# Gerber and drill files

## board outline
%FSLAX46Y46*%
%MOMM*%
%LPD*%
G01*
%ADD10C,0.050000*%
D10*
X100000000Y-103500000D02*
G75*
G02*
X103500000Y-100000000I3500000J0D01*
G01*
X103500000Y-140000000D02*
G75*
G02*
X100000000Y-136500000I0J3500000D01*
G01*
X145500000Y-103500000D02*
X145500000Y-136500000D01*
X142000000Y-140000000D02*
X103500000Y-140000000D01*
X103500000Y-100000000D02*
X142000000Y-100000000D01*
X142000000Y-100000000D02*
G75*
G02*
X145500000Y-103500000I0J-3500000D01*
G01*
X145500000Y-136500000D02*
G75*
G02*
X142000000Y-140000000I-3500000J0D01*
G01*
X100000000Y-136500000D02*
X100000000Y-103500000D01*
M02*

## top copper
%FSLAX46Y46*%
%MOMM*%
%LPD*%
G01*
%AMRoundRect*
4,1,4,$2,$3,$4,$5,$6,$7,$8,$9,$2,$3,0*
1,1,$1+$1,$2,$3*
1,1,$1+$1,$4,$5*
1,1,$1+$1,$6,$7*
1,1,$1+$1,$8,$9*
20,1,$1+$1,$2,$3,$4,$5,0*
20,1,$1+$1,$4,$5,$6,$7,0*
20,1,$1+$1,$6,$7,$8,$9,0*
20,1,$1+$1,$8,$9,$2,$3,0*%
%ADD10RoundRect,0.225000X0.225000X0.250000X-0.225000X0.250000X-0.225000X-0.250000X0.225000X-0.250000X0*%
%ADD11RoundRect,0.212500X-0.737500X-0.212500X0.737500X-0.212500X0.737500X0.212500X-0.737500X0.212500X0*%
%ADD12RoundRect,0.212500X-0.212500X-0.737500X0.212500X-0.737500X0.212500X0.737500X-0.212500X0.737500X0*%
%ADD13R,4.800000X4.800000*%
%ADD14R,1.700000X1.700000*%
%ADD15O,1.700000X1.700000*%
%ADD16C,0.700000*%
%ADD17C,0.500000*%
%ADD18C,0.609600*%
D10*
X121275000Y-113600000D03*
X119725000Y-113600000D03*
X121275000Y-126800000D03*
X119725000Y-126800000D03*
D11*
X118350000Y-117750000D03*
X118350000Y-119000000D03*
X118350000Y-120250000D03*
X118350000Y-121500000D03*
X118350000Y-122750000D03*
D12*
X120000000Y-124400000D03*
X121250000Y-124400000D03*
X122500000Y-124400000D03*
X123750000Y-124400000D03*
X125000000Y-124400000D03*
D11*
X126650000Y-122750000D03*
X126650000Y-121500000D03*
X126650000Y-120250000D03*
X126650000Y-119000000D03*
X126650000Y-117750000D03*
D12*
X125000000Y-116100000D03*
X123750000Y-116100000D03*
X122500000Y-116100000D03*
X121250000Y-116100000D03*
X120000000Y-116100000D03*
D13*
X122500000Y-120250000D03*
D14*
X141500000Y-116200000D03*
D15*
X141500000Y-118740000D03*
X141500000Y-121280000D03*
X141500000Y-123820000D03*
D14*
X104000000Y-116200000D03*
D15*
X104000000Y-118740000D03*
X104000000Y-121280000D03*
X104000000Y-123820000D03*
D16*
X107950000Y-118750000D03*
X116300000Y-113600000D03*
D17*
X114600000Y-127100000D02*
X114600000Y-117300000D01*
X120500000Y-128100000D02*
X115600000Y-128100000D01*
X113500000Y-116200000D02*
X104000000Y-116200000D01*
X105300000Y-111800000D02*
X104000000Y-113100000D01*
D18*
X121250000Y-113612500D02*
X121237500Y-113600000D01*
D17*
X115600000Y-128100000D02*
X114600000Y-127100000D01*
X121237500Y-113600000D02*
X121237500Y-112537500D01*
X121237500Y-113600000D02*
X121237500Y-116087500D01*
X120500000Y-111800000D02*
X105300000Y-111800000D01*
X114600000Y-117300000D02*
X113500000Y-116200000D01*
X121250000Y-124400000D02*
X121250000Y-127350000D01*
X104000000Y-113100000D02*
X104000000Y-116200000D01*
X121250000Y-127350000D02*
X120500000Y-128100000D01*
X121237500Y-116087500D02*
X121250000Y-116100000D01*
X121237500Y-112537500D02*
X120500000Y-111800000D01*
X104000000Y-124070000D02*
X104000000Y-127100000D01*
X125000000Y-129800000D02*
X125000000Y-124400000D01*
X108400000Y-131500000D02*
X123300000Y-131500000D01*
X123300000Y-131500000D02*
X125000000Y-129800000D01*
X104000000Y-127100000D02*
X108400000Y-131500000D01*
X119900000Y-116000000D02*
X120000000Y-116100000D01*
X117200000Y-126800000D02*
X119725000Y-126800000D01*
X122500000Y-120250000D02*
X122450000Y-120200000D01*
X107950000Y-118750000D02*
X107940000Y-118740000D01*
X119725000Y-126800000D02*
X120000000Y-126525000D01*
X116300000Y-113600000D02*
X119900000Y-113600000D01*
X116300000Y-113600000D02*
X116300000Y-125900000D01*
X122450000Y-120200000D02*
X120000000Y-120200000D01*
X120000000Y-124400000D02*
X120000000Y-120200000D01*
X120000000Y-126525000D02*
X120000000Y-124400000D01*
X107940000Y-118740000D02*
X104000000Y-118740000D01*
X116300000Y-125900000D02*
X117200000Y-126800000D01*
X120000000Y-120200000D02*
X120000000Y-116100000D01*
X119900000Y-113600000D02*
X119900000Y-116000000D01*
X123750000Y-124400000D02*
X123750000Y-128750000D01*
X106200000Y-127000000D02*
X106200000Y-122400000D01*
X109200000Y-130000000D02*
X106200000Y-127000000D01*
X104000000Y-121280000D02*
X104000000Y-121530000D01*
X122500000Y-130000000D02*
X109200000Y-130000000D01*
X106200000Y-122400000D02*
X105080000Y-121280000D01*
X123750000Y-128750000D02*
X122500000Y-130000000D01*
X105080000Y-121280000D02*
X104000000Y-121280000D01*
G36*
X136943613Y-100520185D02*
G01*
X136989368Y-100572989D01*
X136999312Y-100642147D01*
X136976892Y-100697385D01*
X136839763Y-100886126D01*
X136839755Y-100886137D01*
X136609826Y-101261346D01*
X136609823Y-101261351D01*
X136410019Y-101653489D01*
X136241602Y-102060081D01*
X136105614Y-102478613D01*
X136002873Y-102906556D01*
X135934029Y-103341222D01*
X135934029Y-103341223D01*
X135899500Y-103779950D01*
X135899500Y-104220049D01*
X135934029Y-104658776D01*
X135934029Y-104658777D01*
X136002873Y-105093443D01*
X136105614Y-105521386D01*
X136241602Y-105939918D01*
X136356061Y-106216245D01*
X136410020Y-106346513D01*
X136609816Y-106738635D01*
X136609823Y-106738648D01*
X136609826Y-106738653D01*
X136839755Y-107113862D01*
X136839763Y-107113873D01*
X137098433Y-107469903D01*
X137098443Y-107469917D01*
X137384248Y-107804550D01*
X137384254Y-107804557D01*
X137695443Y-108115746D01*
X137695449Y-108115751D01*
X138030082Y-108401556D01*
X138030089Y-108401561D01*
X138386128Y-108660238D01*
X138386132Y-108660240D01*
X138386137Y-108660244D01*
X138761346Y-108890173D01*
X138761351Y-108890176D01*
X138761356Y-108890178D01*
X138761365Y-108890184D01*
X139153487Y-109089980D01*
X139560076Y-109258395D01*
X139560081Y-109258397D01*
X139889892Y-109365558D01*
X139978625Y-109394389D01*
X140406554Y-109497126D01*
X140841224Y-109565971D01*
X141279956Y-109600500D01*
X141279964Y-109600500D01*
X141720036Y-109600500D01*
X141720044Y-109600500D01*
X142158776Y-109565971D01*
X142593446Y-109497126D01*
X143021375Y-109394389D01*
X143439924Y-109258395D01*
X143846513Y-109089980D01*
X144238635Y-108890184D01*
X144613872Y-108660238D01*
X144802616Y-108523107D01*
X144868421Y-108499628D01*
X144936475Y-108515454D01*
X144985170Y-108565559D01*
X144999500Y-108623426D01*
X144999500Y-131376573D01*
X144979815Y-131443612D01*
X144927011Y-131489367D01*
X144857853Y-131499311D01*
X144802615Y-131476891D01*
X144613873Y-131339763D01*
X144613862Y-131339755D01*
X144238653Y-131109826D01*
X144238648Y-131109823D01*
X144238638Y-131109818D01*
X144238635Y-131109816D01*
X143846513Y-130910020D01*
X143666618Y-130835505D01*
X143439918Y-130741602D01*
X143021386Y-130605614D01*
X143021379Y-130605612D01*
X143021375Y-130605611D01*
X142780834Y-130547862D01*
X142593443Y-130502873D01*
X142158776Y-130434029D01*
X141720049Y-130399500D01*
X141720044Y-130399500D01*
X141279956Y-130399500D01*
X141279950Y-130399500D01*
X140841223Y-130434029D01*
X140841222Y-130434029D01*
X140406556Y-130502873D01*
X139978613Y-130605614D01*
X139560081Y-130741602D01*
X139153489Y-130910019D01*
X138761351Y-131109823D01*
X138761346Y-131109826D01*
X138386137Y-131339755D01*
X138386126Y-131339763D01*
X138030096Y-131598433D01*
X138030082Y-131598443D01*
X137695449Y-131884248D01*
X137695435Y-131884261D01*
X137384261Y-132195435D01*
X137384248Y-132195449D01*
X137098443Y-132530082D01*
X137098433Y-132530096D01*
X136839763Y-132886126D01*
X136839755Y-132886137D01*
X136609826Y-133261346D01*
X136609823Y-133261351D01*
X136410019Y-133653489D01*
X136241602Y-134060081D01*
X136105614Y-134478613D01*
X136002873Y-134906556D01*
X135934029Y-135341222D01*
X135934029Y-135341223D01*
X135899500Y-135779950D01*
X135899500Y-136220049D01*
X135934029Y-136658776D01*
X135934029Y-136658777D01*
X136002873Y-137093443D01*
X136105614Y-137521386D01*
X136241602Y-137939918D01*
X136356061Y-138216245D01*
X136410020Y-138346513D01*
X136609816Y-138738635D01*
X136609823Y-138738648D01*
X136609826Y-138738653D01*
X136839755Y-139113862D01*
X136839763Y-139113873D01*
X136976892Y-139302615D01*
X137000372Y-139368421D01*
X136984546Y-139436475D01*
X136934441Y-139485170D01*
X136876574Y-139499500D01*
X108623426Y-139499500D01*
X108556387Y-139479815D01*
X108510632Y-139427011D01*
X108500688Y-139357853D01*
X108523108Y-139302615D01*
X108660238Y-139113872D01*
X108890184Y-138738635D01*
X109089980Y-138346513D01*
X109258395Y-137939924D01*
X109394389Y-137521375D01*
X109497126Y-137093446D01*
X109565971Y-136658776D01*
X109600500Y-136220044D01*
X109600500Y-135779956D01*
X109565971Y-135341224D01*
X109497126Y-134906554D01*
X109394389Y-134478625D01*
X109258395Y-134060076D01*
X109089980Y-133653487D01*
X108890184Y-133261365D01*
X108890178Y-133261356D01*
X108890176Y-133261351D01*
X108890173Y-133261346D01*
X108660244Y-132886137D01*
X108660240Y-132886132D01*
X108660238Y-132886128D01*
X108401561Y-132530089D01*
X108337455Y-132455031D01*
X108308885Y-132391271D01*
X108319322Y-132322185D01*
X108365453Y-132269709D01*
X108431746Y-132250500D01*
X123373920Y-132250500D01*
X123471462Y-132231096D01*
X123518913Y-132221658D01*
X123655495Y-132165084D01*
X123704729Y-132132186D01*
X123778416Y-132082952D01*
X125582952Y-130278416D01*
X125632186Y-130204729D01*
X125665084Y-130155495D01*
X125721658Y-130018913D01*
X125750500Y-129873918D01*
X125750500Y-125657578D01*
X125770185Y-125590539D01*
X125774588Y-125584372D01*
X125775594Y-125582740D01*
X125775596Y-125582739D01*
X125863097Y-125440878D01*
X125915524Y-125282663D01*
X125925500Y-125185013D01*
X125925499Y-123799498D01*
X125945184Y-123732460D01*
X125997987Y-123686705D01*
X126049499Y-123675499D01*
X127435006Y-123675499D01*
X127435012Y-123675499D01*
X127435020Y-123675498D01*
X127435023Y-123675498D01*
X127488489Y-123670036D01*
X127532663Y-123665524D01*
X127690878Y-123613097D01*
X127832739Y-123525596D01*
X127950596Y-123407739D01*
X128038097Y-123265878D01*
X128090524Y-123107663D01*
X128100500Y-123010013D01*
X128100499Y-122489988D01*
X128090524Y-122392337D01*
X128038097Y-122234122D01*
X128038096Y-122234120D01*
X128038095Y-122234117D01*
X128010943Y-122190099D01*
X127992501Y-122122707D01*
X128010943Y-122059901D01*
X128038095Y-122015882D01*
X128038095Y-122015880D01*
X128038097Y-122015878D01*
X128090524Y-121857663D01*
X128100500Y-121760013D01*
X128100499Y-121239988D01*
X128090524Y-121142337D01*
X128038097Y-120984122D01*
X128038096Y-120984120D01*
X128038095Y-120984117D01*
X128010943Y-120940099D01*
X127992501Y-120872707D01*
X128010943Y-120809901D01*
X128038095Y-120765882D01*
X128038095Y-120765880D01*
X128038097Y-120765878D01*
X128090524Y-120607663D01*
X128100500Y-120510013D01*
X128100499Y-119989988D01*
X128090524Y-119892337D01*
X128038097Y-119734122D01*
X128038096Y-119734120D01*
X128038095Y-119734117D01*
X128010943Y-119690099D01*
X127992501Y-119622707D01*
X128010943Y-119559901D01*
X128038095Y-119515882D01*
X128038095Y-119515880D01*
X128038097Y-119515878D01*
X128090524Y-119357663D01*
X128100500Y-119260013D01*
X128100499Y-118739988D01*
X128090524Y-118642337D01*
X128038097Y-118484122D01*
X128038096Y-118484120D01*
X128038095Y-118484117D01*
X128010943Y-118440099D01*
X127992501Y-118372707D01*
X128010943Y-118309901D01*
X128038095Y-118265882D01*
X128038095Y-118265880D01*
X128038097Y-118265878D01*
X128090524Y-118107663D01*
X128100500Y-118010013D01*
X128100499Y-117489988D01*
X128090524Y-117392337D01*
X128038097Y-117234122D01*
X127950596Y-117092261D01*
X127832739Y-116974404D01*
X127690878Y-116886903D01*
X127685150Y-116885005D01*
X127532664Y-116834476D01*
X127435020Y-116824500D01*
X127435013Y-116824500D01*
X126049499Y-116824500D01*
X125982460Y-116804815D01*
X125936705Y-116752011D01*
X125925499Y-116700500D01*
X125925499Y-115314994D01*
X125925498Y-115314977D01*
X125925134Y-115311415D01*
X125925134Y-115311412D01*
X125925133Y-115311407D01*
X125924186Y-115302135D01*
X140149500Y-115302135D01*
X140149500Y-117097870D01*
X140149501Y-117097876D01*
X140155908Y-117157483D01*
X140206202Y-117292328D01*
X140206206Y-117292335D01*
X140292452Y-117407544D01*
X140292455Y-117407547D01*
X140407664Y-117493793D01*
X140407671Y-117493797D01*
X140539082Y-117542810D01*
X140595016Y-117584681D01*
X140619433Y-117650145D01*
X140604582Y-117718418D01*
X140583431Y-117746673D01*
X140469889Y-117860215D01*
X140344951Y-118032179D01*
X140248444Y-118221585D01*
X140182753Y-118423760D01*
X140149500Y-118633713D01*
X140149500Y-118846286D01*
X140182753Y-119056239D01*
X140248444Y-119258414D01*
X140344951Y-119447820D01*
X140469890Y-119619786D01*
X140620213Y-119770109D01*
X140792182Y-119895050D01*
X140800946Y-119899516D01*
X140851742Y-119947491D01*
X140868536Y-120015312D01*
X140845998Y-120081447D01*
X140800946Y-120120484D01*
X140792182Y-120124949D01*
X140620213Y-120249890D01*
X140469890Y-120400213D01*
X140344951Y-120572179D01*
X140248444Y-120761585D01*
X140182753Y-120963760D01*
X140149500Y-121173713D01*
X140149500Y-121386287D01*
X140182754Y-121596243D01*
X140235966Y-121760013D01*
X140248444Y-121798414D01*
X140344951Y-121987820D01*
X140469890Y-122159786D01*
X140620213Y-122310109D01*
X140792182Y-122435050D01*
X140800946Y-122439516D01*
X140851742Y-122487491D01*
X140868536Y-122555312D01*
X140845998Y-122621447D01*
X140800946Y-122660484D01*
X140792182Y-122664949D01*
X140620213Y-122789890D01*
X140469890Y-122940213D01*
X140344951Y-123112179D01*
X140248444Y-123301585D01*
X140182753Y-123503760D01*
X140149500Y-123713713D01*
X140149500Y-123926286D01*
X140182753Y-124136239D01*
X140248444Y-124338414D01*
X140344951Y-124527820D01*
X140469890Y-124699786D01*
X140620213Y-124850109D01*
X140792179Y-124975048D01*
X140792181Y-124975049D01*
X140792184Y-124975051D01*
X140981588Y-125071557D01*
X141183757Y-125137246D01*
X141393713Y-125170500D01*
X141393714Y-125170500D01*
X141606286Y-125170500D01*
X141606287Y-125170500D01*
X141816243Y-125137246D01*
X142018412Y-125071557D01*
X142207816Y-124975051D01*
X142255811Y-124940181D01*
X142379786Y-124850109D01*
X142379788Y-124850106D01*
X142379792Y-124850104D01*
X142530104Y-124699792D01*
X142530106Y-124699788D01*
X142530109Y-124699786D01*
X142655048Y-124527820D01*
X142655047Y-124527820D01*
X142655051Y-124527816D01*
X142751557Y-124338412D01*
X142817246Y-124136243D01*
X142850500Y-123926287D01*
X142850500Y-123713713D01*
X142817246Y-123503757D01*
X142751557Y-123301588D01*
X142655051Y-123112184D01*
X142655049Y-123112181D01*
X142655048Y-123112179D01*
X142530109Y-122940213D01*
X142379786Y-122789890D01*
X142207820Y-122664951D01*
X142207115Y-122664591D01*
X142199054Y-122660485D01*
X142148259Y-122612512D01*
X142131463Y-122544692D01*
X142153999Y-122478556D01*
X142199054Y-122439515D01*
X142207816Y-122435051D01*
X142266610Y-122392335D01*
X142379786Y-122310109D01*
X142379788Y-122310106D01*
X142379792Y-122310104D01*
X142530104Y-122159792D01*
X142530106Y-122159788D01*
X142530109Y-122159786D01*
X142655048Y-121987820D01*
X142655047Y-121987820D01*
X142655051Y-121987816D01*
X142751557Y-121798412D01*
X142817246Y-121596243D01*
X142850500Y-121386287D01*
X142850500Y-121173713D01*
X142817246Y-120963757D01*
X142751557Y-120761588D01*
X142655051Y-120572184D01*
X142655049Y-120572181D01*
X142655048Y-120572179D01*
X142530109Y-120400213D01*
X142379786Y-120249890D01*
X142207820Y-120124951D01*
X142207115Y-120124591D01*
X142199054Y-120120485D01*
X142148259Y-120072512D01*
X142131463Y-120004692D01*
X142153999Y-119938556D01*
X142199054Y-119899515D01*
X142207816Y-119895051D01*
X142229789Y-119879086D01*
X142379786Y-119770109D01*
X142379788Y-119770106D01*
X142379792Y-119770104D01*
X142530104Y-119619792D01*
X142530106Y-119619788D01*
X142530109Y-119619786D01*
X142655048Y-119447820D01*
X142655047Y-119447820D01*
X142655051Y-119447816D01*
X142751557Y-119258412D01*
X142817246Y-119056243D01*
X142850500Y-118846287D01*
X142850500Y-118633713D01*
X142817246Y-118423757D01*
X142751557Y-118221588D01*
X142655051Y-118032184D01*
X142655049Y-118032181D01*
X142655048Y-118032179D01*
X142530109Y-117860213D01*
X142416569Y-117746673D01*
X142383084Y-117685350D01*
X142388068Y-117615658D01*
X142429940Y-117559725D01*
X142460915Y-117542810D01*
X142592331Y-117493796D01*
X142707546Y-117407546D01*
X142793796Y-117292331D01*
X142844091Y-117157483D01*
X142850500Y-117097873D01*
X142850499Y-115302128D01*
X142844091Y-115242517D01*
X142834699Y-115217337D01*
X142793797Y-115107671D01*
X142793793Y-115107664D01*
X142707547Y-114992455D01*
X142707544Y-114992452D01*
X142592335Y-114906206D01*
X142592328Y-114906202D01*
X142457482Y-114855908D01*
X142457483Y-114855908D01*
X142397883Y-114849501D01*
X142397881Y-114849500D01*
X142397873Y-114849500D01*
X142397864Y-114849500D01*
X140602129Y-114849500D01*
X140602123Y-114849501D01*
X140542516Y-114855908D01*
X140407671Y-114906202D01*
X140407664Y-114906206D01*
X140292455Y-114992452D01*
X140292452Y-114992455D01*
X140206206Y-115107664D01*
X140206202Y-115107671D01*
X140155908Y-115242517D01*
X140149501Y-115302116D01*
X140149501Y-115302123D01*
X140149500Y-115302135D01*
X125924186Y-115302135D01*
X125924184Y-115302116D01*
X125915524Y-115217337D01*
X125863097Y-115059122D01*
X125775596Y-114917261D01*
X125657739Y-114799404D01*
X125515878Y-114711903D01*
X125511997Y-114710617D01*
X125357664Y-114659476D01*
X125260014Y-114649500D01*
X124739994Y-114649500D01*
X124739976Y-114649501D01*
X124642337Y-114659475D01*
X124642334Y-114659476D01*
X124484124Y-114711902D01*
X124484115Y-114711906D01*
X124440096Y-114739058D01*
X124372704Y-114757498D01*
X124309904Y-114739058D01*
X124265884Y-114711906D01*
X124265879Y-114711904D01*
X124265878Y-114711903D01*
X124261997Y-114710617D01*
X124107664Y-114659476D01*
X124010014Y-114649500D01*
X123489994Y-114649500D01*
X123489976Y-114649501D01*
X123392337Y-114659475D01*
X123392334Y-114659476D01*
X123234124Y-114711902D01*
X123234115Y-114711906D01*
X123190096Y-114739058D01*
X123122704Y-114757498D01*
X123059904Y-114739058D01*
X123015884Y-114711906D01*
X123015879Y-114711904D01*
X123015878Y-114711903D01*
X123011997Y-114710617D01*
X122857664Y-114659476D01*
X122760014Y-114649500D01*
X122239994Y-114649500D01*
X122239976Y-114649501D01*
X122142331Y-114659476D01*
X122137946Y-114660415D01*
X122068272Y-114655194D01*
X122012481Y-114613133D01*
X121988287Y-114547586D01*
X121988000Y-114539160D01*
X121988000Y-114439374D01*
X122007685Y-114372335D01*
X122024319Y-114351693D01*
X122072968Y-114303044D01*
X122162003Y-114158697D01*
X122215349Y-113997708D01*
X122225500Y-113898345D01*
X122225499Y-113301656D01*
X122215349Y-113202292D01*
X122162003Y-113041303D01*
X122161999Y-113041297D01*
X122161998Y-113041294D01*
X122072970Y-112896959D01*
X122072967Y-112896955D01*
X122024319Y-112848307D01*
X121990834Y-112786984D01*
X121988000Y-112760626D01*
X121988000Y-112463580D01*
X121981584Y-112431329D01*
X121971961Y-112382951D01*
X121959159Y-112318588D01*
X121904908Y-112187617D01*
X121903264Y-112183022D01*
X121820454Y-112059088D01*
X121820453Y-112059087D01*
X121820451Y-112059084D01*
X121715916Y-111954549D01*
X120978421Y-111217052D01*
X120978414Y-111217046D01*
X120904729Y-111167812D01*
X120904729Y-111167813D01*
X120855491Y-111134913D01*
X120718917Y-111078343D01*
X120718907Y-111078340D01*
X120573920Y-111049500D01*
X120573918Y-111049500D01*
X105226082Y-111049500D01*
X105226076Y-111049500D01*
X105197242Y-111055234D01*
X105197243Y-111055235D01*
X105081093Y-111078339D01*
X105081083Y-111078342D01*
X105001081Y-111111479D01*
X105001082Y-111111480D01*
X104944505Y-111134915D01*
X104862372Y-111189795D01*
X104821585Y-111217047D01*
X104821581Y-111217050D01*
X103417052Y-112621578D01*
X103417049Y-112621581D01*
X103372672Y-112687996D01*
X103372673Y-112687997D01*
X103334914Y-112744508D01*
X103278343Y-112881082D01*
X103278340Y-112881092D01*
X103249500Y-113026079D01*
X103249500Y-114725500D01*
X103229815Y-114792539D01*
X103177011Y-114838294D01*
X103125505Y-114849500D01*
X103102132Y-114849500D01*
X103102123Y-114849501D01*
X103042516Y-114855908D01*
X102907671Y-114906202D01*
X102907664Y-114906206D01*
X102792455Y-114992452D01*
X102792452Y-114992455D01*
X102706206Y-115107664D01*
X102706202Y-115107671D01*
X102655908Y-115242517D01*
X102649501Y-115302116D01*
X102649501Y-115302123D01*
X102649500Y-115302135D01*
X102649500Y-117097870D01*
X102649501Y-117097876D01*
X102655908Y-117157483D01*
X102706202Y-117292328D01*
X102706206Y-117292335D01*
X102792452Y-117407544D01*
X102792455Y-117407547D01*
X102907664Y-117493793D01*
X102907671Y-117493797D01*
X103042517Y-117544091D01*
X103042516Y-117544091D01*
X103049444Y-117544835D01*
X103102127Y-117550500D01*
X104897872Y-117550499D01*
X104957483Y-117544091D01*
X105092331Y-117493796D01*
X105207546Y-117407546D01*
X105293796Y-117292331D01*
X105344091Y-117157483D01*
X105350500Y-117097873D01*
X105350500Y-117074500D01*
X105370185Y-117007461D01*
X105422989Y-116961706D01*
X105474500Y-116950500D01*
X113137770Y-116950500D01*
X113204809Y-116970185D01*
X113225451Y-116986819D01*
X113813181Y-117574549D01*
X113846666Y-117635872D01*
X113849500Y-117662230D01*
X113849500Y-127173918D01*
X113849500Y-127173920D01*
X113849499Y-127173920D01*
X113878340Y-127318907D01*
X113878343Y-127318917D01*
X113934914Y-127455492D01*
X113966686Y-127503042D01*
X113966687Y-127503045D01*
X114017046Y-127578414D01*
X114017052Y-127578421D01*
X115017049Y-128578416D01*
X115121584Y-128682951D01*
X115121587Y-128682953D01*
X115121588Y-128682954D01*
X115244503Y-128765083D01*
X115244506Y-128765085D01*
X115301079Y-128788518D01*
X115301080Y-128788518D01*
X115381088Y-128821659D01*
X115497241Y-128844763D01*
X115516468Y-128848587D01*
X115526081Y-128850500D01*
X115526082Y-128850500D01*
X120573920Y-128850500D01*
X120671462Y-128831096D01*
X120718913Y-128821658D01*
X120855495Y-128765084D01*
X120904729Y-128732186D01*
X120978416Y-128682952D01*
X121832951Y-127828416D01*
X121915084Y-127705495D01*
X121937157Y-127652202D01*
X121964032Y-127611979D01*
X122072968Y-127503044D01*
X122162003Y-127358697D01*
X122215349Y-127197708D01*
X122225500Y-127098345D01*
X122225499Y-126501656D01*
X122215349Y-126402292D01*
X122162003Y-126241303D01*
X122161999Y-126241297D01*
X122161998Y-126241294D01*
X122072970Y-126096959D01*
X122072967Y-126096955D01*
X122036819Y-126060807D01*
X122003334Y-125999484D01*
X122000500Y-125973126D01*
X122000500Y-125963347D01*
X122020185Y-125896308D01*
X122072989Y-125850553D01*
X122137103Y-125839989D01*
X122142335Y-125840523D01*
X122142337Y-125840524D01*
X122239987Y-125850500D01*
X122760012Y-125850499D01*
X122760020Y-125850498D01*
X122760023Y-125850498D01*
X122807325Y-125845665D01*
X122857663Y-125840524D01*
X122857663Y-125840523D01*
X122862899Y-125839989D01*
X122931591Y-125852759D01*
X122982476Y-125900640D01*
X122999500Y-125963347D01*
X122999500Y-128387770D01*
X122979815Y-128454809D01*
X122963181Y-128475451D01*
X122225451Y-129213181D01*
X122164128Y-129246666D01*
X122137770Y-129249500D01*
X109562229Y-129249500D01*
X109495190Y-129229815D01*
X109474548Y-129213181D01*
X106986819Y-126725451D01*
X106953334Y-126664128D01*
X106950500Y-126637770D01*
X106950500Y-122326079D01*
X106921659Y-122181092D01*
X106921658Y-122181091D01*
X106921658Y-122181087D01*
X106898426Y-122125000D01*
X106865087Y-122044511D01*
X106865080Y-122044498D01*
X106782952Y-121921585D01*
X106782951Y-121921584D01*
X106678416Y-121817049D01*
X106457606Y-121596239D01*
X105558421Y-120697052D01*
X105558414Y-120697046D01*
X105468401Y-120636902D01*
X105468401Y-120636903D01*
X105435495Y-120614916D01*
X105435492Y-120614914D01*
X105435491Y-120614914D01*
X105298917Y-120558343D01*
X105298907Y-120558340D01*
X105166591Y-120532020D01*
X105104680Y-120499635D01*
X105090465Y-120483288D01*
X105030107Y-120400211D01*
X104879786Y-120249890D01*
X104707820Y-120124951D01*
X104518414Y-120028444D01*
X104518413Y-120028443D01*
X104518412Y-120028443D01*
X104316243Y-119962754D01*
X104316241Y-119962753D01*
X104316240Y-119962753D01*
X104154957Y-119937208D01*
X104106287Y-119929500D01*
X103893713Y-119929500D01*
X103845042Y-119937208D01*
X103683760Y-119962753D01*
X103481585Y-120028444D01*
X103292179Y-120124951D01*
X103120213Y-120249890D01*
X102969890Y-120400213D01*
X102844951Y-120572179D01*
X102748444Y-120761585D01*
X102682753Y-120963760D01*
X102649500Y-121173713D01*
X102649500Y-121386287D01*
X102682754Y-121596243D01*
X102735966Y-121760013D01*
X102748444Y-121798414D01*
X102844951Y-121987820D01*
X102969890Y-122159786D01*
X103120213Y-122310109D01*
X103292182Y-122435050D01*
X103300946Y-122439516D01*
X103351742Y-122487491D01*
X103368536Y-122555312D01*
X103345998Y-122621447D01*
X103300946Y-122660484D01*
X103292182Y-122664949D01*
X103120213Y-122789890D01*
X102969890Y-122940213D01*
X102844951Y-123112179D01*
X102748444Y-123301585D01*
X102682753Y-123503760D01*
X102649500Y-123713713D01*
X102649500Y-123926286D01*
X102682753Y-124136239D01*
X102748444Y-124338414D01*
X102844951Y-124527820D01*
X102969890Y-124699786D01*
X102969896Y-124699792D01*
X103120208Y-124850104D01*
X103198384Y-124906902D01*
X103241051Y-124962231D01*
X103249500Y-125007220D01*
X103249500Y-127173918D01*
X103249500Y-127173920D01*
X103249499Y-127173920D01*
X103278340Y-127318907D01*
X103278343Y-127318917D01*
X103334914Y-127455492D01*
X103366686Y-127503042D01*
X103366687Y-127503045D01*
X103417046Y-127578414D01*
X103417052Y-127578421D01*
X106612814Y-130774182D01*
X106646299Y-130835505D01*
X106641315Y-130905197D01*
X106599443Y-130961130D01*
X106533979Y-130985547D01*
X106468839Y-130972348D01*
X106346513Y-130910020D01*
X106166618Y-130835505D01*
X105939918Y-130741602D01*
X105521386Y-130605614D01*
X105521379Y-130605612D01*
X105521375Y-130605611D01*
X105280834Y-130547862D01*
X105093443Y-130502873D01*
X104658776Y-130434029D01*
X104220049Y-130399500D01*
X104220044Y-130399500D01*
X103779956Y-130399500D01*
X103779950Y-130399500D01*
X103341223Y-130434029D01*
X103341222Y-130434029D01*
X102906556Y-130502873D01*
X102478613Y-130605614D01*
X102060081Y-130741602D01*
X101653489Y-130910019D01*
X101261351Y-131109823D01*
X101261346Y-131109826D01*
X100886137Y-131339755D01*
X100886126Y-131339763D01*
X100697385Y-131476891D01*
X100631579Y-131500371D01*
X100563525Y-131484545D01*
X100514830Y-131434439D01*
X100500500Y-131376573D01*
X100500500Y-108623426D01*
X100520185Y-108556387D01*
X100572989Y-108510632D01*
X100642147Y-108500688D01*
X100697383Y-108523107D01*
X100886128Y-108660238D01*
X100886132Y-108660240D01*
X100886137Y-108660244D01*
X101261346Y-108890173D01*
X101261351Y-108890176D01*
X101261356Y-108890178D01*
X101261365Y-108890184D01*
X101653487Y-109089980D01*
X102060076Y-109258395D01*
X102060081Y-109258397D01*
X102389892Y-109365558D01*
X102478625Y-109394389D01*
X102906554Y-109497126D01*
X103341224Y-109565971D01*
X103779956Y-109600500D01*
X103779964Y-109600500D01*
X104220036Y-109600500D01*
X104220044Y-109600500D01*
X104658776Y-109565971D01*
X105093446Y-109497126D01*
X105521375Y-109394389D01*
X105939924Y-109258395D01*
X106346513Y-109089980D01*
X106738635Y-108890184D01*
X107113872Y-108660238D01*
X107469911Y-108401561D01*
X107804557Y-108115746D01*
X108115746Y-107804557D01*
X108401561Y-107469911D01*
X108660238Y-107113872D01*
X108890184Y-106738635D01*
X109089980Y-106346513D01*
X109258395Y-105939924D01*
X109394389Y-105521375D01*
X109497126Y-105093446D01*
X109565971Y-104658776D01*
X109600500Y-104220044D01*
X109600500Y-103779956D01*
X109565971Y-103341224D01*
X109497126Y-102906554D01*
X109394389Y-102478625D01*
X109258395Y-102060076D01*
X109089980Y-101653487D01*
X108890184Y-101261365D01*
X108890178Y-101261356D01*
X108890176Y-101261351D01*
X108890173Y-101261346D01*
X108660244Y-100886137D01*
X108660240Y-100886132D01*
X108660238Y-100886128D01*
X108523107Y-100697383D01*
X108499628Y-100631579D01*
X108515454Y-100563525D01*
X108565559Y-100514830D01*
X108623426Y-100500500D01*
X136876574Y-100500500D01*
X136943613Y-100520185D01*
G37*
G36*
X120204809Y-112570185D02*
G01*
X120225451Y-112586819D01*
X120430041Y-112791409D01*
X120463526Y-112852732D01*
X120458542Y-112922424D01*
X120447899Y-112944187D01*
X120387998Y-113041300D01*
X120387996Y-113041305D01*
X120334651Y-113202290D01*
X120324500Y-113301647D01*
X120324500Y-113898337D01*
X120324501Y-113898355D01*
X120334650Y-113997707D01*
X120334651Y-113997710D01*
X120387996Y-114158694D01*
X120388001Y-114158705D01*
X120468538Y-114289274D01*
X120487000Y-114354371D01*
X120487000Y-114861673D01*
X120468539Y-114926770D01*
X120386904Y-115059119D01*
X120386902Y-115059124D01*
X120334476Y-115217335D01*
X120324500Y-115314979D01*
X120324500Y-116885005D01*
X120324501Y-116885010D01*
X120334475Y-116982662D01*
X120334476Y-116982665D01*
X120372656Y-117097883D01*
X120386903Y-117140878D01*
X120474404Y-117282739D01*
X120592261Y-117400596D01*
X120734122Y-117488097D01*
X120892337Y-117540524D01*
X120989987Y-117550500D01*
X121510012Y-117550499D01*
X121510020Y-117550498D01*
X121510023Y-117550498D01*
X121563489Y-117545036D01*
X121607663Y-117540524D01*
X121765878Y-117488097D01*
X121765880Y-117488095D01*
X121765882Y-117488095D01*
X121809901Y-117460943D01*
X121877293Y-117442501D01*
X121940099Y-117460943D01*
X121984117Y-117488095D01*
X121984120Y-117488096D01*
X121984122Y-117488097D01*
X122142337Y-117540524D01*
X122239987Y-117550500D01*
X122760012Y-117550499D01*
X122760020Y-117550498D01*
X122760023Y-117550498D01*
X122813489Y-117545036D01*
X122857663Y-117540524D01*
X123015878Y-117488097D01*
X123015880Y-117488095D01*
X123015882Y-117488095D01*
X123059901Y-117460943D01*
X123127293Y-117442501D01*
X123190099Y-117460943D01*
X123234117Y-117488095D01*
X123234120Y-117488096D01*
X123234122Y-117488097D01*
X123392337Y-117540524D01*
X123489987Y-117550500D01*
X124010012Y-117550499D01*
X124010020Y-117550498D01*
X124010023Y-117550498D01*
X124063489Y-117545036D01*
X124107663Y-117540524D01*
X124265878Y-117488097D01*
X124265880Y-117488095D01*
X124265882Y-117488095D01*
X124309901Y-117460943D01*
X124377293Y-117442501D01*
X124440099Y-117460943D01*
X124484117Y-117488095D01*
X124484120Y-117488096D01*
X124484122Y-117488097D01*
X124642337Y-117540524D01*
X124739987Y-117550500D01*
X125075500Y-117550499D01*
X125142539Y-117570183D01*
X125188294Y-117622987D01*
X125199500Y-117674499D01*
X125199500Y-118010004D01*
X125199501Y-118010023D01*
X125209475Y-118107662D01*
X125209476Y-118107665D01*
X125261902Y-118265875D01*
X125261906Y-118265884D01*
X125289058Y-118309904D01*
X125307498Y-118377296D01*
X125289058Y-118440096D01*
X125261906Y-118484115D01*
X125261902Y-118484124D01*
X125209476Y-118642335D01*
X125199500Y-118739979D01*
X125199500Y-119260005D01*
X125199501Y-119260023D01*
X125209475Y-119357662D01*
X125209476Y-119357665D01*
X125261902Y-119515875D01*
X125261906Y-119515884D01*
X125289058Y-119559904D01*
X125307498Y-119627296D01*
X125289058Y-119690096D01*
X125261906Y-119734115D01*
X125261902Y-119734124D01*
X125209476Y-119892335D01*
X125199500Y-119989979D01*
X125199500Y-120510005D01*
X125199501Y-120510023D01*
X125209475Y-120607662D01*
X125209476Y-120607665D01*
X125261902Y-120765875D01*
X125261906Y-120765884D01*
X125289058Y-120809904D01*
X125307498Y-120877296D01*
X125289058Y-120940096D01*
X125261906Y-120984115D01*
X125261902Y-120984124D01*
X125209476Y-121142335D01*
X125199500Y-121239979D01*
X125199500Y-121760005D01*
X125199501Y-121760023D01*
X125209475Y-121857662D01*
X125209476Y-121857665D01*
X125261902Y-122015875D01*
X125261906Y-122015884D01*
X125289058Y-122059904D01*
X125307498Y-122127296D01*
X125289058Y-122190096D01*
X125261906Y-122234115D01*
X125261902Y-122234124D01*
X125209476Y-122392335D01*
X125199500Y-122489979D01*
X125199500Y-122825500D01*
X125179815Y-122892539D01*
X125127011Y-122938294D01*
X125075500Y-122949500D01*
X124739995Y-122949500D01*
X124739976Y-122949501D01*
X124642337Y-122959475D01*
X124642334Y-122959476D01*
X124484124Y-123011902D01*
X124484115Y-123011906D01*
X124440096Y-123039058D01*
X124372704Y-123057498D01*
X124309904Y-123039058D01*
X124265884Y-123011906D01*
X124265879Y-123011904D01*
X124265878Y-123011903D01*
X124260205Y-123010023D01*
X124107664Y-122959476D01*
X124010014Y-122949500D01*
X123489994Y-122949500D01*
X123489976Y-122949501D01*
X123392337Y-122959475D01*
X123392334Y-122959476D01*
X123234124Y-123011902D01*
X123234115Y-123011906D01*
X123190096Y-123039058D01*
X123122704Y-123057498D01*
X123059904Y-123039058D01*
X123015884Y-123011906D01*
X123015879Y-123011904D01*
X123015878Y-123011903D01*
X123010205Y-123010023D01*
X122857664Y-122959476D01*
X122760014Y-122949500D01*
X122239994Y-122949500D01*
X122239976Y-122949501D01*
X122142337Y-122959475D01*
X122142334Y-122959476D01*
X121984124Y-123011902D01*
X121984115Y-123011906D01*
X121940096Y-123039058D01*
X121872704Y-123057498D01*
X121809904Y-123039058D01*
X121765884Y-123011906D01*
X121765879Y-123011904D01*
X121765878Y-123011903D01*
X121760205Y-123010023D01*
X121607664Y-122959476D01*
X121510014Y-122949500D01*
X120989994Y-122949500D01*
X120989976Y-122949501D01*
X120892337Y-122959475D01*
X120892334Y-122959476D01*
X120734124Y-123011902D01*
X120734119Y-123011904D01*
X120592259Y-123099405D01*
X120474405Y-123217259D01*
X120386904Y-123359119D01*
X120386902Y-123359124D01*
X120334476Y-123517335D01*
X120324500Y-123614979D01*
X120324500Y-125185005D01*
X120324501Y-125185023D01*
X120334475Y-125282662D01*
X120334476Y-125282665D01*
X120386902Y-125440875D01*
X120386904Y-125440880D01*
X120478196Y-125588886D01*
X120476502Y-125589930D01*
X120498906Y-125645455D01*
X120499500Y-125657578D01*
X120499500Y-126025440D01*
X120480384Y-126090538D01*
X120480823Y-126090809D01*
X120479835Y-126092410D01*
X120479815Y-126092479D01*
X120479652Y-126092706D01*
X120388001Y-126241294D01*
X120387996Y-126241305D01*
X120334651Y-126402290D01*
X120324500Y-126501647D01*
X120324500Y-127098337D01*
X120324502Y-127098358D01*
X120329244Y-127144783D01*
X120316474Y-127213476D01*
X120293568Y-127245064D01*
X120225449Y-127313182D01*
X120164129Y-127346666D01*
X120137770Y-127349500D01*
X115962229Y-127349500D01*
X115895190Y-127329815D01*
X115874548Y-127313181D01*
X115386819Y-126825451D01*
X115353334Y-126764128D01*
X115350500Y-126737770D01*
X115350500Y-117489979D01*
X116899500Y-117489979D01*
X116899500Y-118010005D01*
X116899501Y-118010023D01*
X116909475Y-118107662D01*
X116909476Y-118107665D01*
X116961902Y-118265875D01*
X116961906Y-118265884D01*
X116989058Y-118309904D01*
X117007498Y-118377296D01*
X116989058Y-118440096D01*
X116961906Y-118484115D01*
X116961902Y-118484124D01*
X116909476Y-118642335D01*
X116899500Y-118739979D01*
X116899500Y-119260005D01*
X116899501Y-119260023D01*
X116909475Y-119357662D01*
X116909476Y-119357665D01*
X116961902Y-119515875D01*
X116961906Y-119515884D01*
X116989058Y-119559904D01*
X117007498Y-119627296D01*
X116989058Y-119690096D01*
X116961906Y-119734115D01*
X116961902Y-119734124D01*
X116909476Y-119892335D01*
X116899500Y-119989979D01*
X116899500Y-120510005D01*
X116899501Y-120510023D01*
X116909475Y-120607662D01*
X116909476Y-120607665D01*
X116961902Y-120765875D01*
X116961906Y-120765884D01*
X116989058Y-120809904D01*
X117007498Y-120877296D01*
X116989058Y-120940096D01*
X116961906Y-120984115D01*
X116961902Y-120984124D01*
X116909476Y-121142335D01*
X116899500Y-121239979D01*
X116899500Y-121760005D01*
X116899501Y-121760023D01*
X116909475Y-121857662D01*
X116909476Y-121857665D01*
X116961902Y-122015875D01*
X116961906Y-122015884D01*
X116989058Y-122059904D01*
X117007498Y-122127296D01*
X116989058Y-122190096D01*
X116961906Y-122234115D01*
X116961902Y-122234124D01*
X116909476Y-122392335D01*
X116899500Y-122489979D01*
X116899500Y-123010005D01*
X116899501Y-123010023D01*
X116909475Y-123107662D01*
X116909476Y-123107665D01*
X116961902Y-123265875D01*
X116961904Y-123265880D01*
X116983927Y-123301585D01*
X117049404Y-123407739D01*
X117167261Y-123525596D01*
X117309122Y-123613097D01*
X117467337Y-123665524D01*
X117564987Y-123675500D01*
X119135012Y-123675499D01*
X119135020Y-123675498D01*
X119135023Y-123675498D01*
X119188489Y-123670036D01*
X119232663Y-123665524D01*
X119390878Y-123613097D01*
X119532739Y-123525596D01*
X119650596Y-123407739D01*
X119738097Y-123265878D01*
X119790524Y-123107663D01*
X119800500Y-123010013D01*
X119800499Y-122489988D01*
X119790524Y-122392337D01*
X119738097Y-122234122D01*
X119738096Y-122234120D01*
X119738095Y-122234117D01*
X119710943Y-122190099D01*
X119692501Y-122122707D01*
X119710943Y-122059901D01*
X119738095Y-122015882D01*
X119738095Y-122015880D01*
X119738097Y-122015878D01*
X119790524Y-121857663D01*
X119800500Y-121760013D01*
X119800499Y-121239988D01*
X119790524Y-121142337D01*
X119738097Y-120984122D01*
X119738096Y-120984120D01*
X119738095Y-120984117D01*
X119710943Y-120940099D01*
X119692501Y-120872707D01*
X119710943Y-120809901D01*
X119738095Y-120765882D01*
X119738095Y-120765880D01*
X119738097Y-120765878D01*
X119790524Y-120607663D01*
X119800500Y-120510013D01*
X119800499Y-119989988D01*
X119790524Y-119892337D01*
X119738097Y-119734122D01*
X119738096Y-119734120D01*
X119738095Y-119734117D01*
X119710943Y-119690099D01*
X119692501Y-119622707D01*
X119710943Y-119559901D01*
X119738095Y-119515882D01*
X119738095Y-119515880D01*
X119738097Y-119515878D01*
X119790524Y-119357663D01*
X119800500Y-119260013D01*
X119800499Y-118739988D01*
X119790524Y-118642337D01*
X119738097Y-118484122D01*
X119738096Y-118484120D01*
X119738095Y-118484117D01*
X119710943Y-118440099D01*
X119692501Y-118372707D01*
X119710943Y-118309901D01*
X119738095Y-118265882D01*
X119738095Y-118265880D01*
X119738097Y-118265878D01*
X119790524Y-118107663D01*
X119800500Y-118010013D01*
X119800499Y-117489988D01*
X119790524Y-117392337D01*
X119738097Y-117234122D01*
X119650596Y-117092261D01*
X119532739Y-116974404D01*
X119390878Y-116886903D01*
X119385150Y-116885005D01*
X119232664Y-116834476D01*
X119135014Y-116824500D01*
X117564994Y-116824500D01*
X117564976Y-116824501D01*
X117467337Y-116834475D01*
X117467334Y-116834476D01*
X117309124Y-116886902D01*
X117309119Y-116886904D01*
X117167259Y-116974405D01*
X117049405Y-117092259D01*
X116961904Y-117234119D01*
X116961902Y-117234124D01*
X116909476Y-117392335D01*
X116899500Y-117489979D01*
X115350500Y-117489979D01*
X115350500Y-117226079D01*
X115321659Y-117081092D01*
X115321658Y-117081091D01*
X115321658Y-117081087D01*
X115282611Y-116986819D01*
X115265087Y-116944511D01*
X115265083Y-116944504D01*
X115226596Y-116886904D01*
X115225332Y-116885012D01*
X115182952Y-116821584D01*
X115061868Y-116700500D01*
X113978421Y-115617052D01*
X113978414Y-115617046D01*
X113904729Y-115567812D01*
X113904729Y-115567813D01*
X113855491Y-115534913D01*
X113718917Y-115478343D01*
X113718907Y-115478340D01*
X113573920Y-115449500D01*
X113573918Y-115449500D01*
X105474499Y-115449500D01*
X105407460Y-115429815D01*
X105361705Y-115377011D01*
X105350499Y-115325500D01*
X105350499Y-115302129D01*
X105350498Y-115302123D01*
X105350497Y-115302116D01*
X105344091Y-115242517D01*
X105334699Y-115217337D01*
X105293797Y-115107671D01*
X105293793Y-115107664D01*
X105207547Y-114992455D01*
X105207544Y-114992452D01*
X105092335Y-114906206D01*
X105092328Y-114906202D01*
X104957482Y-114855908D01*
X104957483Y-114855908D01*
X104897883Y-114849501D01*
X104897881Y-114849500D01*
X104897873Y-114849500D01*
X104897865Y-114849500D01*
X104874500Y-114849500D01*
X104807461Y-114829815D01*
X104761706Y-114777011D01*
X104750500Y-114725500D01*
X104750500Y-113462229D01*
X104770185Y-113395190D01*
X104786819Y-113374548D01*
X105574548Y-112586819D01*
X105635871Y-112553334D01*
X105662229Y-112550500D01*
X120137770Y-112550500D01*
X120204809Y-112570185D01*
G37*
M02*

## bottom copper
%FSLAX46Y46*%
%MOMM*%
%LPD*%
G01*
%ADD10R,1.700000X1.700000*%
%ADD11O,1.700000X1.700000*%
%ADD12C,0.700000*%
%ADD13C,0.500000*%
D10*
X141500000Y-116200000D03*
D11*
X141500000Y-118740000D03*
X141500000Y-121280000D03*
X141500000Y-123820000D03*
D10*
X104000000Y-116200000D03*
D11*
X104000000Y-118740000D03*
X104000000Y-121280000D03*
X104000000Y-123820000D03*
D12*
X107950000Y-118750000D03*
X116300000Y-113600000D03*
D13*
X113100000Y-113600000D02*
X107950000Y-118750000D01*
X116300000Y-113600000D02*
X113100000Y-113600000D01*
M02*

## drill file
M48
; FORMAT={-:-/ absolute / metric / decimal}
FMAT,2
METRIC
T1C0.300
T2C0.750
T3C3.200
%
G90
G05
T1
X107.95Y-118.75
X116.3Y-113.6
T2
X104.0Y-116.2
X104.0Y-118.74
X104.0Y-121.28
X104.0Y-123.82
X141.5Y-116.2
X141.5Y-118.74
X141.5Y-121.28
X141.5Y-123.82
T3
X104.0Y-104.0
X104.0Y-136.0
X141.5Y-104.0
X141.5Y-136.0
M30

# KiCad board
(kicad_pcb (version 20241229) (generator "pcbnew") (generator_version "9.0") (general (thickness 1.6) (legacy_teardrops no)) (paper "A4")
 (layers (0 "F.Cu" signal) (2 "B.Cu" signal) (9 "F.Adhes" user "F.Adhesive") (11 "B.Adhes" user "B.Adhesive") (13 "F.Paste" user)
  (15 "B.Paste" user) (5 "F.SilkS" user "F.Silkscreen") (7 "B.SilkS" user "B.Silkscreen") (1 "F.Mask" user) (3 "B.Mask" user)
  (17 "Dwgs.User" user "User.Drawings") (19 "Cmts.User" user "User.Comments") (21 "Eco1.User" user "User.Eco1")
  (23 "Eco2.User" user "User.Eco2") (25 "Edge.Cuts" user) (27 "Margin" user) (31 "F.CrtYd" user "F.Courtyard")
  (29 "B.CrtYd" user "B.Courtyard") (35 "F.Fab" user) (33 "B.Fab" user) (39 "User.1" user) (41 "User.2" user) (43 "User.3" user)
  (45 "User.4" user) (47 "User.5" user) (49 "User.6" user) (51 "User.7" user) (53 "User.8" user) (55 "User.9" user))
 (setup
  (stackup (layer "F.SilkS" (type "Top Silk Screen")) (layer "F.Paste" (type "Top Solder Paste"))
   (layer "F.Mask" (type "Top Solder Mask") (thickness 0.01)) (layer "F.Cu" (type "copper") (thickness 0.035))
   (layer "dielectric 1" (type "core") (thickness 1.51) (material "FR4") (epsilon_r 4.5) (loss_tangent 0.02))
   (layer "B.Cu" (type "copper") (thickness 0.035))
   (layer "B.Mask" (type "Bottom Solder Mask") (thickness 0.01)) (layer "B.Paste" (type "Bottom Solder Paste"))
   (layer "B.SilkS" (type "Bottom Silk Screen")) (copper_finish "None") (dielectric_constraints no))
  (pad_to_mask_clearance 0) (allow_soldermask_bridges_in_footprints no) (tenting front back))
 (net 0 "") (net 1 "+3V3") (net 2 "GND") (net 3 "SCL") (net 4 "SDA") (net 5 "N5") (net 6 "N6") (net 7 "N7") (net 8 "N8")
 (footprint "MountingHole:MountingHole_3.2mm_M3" (layer "F.Cu") (at 141.5 104)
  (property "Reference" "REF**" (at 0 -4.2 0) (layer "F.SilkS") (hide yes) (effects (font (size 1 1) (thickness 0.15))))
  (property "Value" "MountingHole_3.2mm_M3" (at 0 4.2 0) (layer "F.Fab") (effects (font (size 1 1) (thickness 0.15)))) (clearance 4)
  (pad "" np_thru_hole circle (at 0 0) (size 3.2 3.2) (drill 3.2) (layers "*.Cu" "*.Mask")))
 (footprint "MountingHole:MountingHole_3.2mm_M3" (layer "F.Cu") (at 141.5 136)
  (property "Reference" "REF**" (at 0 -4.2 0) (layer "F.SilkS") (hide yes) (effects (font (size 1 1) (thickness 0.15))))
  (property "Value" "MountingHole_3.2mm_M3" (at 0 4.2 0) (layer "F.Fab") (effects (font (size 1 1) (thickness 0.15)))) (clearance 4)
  (pad "" np_thru_hole circle (at 0 0) (size 3.2 3.2) (drill 3.2) (layers "*.Cu" "*.Mask")))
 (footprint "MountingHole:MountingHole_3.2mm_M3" (layer "F.Cu") (at 104 104)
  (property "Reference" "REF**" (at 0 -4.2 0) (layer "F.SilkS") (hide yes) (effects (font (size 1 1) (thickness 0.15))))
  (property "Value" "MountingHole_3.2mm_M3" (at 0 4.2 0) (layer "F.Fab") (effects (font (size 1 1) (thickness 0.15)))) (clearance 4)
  (pad "" np_thru_hole circle (at 0 0) (size 3.2 3.2) (drill 3.2) (layers "*.Cu" "*.Mask")))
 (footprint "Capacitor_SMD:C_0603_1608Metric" (layer "F.Cu") (at 120.5 113.6 180)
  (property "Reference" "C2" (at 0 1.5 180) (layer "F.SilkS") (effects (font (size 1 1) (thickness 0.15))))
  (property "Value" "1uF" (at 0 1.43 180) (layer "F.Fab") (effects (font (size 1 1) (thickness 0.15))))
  (pad "1" smd roundrect (at -0.775 0 180) (size 0.9 0.95) (layers "F.Cu" "F.Mask" "F.Paste") (roundrect_rratio 0.25) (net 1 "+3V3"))
  (pad "2" smd roundrect (at 0.775 0 180) (size 0.9 0.95) (layers "F.Cu" "F.Mask" "F.Paste") (roundrect_rratio 0.25) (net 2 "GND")))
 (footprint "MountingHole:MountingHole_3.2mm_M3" (layer "F.Cu") (at 104 136)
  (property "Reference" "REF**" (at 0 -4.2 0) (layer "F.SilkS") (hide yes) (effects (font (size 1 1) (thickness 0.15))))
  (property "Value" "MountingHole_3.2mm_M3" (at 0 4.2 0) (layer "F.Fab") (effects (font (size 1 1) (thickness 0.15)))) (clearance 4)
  (pad "" np_thru_hole circle (at 0 0) (size 3.2 3.2) (drill 3.2) (layers "*.Cu" "*.Mask")))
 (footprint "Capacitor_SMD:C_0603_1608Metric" (layer "F.Cu") (at 120.5 126.8 180)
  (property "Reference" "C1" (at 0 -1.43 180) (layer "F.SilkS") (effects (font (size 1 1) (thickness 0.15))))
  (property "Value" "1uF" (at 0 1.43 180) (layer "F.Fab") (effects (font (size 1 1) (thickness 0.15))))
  (pad "1" smd roundrect (at -0.775 0 180) (size 0.9 0.95) (layers "F.Cu" "F.Mask" "F.Paste") (roundrect_rratio 0.25) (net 1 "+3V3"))
  (pad "2" smd roundrect (at 0.775 0 180) (size 0.9 0.95) (layers "F.Cu" "F.Mask" "F.Paste") (roundrect_rratio 0.25) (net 2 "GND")))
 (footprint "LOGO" (layer "F.Cu") (at 134.459805 120.26479)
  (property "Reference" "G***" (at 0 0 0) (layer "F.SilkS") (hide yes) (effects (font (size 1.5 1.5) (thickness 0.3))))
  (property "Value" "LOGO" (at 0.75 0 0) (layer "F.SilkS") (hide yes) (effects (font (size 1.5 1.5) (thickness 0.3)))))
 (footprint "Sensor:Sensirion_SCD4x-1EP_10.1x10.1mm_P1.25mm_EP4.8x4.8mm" (layer "F.Cu") (at 122.5 120.25)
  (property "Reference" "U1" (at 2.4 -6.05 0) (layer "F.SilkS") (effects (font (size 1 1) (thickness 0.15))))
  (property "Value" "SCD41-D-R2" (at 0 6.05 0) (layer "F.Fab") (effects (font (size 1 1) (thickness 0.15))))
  (pad "" smd roundrect (at -1.2 -1.2) (size 1.93 1.93) (layers "F.Paste") (roundrect_rratio 0.129534))
  (pad "" smd roundrect (at -1.2 1.2) (size 1.93 1.93) (layers "F.Paste") (roundrect_rratio 0.129534))
  (pad "" smd roundrect (at 1.2 -1.2) (size 1.93 1.93) (layers "F.Paste") (roundrect_rratio 0.129534))
  (pad "" smd roundrect (at 1.2 1.2) (size 1.93 1.93) (layers "F.Paste") (roundrect_rratio 0.129534))
  (pad "1" smd roundrect (at -4.15 -2.5) (size 1.9 0.85) (layers "F.Cu" "F.Mask" "F.Paste") (roundrect_rratio 0.25))
  (pad "2" smd roundrect (at -4.15 -1.25) (size 1.9 0.85) (layers "F.Cu" "F.Mask" "F.Paste") (roundrect_rratio 0.25))
  (pad "3" smd roundrect (at -4.15 0) (size 1.9 0.85) (layers "F.Cu" "F.Mask" "F.Paste") (roundrect_rratio 0.25))
  (pad "4" smd roundrect (at -4.15 1.25) (size 1.9 0.85) (layers "F.Cu" "F.Mask" "F.Paste") (roundrect_rratio 0.25))
  (pad "5" smd roundrect (at -4.15 2.5) (size 1.9 0.85) (layers "F.Cu" "F.Mask" "F.Paste") (roundrect_rratio 0.25))
  (pad "6" smd roundrect (at -2.5 4.15) (size 0.85 1.9) (layers "F.Cu" "F.Mask" "F.Paste") (roundrect_rratio 0.25) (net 2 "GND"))
  (pad "7" smd roundrect (at -1.25 4.15) (size 0.85 1.9) (layers "F.Cu" "F.Mask" "F.Paste") (roundrect_rratio 0.25) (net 1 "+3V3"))
  (pad "8" smd roundrect (at 0 4.15) (size 0.85 1.9) (layers "F.Cu" "F.Mask" "F.Paste") (roundrect_rratio 0.25))
  (pad "9" smd roundrect (at 1.25 4.15) (size 0.85 1.9) (layers "F.Cu" "F.Mask" "F.Paste") (roundrect_rratio 0.25) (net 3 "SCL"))
  (pad "10" smd roundrect (at 2.5 4.15) (size 0.85 1.9) (layers "F.Cu" "F.Mask" "F.Paste") (roundrect_rratio 0.25) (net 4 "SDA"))
  (pad "11" smd roundrect (at 4.15 2.5) (size 1.9 0.85) (layers "F.Cu" "F.Mask" "F.Paste") (roundrect_rratio 0.25))
  (pad "12" smd roundrect (at 4.15 1.25) (size 1.9 0.85) (layers "F.Cu" "F.Mask" "F.Paste") (roundrect_rratio 0.25))
  (pad "13" smd roundrect (at 4.15 0) (size 1.9 0.85) (layers "F.Cu" "F.Mask" "F.Paste") (roundrect_rratio 0.25))
  (pad "14" smd roundrect (at 4.15 -1.25) (size 1.9 0.85) (layers "F.Cu" "F.Mask" "F.Paste") (roundrect_rratio 0.25))
  (pad "15" smd roundrect (at 4.15 -2.5) (size 1.9 0.85) (layers "F.Cu" "F.Mask" "F.Paste") (roundrect_rratio 0.25))
  (pad "16" smd roundrect (at 2.5 -4.15) (size 0.85 1.9) (layers "F.Cu" "F.Mask" "F.Paste") (roundrect_rratio 0.25))
  (pad "17" smd roundrect (at 1.25 -4.15) (size 0.85 1.9) (layers "F.Cu" "F.Mask" "F.Paste") (roundrect_rratio 0.25))
  (pad "18" smd roundrect (at 0 -4.15) (size 0.85 1.9) (layers "F.Cu" "F.Mask" "F.Paste") (roundrect_rratio 0.25))
  (pad "19" smd roundrect (at -1.25 -4.15) (size 0.85 1.9) (layers "F.Cu" "F.Mask" "F.Paste") (roundrect_rratio 0.25) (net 1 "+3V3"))
  (pad "20" smd roundrect (at -2.5 -4.15) (size 0.85 1.9) (layers "F.Cu" "F.Mask" "F.Paste") (roundrect_rratio 0.25) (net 2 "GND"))
  (pad "21" smd rect (at 0 0) (size 4.8 4.8) (layers "F.Cu" "F.Mask") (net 2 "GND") (zone_connect 2)))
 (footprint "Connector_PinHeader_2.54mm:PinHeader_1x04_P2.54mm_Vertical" (layer "B.Cu") (at 141.5 116.2 180)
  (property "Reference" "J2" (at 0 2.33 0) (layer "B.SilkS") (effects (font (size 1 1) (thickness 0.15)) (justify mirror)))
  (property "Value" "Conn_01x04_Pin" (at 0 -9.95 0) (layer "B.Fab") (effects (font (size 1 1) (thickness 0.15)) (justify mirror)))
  (pad "1" thru_hole rect (at 0 0 180) (size 1.7 1.7) (drill 0.75) (layers "*.Cu" "*.Mask") (remove_unused_layers no) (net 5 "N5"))
  (pad "2" thru_hole oval (at 0 -2.54 180) (size 1.7 1.7) (drill 0.75) (layers "*.Cu" "*.Mask") (remove_unused_layers no) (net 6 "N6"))
  (pad "3" thru_hole oval (at 0 -5.08 180) (size 1.7 1.7) (drill 0.75) (layers "*.Cu" "*.Mask") (remove_unused_layers no) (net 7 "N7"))
  (pad "4" thru_hole oval (at 0 -7.62 180) (size 1.7 1.7) (drill 0.75) (layers "*.Cu" "*.Mask") (remove_unused_layers no) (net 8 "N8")))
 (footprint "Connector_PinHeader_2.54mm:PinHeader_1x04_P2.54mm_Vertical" (layer "B.Cu") (at 104 116.2 180)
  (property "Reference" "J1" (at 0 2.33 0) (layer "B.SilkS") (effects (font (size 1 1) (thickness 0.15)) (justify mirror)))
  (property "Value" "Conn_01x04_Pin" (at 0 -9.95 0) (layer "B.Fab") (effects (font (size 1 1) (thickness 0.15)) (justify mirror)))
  (pad "1" thru_hole rect (at 0 0 180) (size 1.7 1.7) (drill 0.75) (layers "*.Cu" "*.Mask") (remove_unused_layers no) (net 1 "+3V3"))
  (pad "2" thru_hole oval (at 0 -2.54 180) (size 1.7 1.7) (drill 0.75) (layers "*.Cu" "*.Mask") (remove_unused_layers no) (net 2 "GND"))
  (pad "3" thru_hole oval (at 0 -5.08 180) (size 1.7 1.7) (drill 0.75) (layers "*.Cu" "*.Mask") (remove_unused_layers no) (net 3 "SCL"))
  (pad "4" thru_hole oval (at 0 -7.62 180) (size 1.7 1.7) (drill 0.75) (layers "*.Cu" "*.Mask") (remove_unused_layers no) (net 4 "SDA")))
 (gr_arc (start 100 103.5) (mid 101.025126 101.025126) (end 103.5 100) (stroke (width 0.05) (type default)) (layer "Edge.Cuts"))
 (gr_arc (start 103.5 140) (mid 101.025126 138.974874) (end 100 136.5) (stroke (width 0.05) (type default)) (layer "Edge.Cuts"))
 (gr_line (start 145.5 103.5) (end 145.5 136.5) (stroke (width 0.05) (type default)) (layer "Edge.Cuts"))
 (gr_line (start 142 140) (end 103.5 140) (stroke (width 0.05) (type default)) (layer "Edge.Cuts"))
 (gr_line (start 103.5 100) (end 142 100) (stroke (width 0.05) (type default)) (layer "Edge.Cuts"))
 (gr_arc (start 142 100) (mid 144.474874 101.025126) (end 145.5 103.5) (stroke (width 0.05) (type default)) (layer "Edge.Cuts"))
 (gr_arc (start 145.5 136.5) (mid 144.474874 138.974874) (end 142 140) (stroke (width 0.05) (type default)) (layer "Edge.Cuts"))
 (gr_line (start 100 136.5) (end 100 103.5) (stroke (width 0.05) (type default)) (layer "Edge.Cuts"))
 (segment (start 114.6 127.1) (end 114.6 117.3) (width 0.5) (layer "F.Cu") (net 1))
 (segment (start 120.5 128.1) (end 115.6 128.1) (width 0.5) (layer "F.Cu") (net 1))
 (segment (start 113.5 116.2) (end 104 116.2) (width 0.5) (layer "F.Cu") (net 1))
 (segment (start 105.3 111.8) (end 104 113.1) (width 0.5) (layer "F.Cu") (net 1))
 (segment (start 121.25 113.6125) (end 121.2375 113.6) (width 0.6096) (layer "F.Cu") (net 1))
 (segment (start 115.6 128.1) (end 114.6 127.1) (width 0.5) (layer "F.Cu") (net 1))
 (segment (start 121.2375 113.6) (end 121.2375 112.5375) (width 0.5) (layer "F.Cu") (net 1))
 (segment (start 121.2375 113.6) (end 121.2375 116.0875) (width 0.5) (layer "F.Cu") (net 1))
 (segment (start 120.5 111.8) (end 105.3 111.8) (width 0.5) (layer "F.Cu") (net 1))
 (segment (start 114.6 117.3) (end 113.5 116.2) (width 0.5) (layer "F.Cu") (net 1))
 (segment (start 121.25 124.4) (end 121.25 127.35) (width 0.5) (layer "F.Cu") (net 1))
 (segment (start 104 113.1) (end 104 116.2) (width 0.5) (layer "F.Cu") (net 1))
 (segment (start 121.25 127.35) (end 120.5 128.1) (width 0.5) (layer "F.Cu") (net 1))
 (segment (start 121.2375 116.0875) (end 121.25 116.1) (width 0.5) (layer "F.Cu") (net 1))
 (segment (start 121.2375 112.5375) (end 120.5 111.8) (width 0.5) (layer "F.Cu") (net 1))
 (segment (start 104 124.07) (end 104 127.1) (width 0.5) (layer "F.Cu") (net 4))
 (segment (start 125 129.8) (end 125 124.4) (width 0.5) (layer "F.Cu") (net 4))
 (segment (start 108.4 131.5) (end 123.3 131.5) (width 0.5) (layer "F.Cu") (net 4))
 (segment (start 123.3 131.5) (end 125 129.8) (width 0.5) (layer "F.Cu") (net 4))
 (segment (start 104 127.1) (end 108.4 131.5) (width 0.5) (layer "F.Cu") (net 4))
 (segment (start 119.9 116) (end 120 116.1) (width 0.5) (layer "F.Cu") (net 2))
 (segment (start 117.2 126.8) (end 119.725 126.8) (width 0.5) (layer "F.Cu") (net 2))
 (segment (start 122.5 120.25) (end 122.45 120.2) (width 0.5) (layer "F.Cu") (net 2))
 (segment (start 107.95 118.75) (end 107.94 118.74) (width 0.5) (layer "F.Cu") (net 2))
 (segment (start 119.725 126.8) (end 120 126.525) (width 0.5) (layer "F.Cu") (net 2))
 (segment (start 116.3 113.6) (end 119.9 113.6) (width 0.5) (layer "F.Cu") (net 2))
 (segment (start 116.3 113.6) (end 116.3 125.9) (width 0.5) (layer "F.Cu") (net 2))
 (segment (start 122.45 120.2) (end 120 120.2) (width 0.5) (layer "F.Cu") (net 2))
 (segment (start 120 124.4) (end 120 120.2) (width 0.5) (layer "F.Cu") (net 2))
 (segment (start 120 126.525) (end 120 124.4) (width 0.5) (layer "F.Cu") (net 2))
 (segment (start 107.94 118.74) (end 104 118.74) (width 0.5) (layer "F.Cu") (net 2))
 (segment (start 116.3 125.9) (end 117.2 126.8) (width 0.5) (layer "F.Cu") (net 2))
 (segment (start 120 120.2) (end 120 116.1) (width 0.5) (layer "F.Cu") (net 2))
 (segment (start 119.9 113.6) (end 119.9 116) (width 0.5) (layer "F.Cu") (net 2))
 (via (at 107.95 118.75) (size 0.7) (drill 0.3) (layers "F.Cu" "B.Cu") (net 2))
 (via (at 116.3 113.6) (size 0.7) (drill 0.3) (layers "F.Cu" "B.Cu") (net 2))
 (segment (start 113.1 113.6) (end 107.95 118.75) (width 0.5) (layer "B.Cu") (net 2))
 (segment (start 116.3 113.6) (end 113.1 113.6) (width 0.5) (layer "B.Cu") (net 2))
 (segment (start 123.75 124.4) (end 123.75 128.75) (width 0.5) (layer "F.Cu") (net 3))
 (segment (start 106.2 127) (end 106.2 122.4) (width 0.5) (layer "F.Cu") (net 3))
 (segment (start 109.2 130) (end 106.2 127) (width 0.5) (layer "F.Cu") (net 3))
 (segment (start 104 121.28) (end 104 121.53) (width 0.5) (layer "F.Cu") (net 3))
 (segment (start 122.5 130) (end 109.2 130) (width 0.5) (layer "F.Cu") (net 3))
 (segment (start 106.2 122.4) (end 105.08 121.28) (width 0.5) (layer "F.Cu") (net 3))
 (segment (start 123.75 128.75) (end 122.5 130) (width 0.5) (layer "F.Cu") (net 3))
 (segment (start 105.08 121.28) (end 104 121.28) (width 0.5) (layer "F.Cu") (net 3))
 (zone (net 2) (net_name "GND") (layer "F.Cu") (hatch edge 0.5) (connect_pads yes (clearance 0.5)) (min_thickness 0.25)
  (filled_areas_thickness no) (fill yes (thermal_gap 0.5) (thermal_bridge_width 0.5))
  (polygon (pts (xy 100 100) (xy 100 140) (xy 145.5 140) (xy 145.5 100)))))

